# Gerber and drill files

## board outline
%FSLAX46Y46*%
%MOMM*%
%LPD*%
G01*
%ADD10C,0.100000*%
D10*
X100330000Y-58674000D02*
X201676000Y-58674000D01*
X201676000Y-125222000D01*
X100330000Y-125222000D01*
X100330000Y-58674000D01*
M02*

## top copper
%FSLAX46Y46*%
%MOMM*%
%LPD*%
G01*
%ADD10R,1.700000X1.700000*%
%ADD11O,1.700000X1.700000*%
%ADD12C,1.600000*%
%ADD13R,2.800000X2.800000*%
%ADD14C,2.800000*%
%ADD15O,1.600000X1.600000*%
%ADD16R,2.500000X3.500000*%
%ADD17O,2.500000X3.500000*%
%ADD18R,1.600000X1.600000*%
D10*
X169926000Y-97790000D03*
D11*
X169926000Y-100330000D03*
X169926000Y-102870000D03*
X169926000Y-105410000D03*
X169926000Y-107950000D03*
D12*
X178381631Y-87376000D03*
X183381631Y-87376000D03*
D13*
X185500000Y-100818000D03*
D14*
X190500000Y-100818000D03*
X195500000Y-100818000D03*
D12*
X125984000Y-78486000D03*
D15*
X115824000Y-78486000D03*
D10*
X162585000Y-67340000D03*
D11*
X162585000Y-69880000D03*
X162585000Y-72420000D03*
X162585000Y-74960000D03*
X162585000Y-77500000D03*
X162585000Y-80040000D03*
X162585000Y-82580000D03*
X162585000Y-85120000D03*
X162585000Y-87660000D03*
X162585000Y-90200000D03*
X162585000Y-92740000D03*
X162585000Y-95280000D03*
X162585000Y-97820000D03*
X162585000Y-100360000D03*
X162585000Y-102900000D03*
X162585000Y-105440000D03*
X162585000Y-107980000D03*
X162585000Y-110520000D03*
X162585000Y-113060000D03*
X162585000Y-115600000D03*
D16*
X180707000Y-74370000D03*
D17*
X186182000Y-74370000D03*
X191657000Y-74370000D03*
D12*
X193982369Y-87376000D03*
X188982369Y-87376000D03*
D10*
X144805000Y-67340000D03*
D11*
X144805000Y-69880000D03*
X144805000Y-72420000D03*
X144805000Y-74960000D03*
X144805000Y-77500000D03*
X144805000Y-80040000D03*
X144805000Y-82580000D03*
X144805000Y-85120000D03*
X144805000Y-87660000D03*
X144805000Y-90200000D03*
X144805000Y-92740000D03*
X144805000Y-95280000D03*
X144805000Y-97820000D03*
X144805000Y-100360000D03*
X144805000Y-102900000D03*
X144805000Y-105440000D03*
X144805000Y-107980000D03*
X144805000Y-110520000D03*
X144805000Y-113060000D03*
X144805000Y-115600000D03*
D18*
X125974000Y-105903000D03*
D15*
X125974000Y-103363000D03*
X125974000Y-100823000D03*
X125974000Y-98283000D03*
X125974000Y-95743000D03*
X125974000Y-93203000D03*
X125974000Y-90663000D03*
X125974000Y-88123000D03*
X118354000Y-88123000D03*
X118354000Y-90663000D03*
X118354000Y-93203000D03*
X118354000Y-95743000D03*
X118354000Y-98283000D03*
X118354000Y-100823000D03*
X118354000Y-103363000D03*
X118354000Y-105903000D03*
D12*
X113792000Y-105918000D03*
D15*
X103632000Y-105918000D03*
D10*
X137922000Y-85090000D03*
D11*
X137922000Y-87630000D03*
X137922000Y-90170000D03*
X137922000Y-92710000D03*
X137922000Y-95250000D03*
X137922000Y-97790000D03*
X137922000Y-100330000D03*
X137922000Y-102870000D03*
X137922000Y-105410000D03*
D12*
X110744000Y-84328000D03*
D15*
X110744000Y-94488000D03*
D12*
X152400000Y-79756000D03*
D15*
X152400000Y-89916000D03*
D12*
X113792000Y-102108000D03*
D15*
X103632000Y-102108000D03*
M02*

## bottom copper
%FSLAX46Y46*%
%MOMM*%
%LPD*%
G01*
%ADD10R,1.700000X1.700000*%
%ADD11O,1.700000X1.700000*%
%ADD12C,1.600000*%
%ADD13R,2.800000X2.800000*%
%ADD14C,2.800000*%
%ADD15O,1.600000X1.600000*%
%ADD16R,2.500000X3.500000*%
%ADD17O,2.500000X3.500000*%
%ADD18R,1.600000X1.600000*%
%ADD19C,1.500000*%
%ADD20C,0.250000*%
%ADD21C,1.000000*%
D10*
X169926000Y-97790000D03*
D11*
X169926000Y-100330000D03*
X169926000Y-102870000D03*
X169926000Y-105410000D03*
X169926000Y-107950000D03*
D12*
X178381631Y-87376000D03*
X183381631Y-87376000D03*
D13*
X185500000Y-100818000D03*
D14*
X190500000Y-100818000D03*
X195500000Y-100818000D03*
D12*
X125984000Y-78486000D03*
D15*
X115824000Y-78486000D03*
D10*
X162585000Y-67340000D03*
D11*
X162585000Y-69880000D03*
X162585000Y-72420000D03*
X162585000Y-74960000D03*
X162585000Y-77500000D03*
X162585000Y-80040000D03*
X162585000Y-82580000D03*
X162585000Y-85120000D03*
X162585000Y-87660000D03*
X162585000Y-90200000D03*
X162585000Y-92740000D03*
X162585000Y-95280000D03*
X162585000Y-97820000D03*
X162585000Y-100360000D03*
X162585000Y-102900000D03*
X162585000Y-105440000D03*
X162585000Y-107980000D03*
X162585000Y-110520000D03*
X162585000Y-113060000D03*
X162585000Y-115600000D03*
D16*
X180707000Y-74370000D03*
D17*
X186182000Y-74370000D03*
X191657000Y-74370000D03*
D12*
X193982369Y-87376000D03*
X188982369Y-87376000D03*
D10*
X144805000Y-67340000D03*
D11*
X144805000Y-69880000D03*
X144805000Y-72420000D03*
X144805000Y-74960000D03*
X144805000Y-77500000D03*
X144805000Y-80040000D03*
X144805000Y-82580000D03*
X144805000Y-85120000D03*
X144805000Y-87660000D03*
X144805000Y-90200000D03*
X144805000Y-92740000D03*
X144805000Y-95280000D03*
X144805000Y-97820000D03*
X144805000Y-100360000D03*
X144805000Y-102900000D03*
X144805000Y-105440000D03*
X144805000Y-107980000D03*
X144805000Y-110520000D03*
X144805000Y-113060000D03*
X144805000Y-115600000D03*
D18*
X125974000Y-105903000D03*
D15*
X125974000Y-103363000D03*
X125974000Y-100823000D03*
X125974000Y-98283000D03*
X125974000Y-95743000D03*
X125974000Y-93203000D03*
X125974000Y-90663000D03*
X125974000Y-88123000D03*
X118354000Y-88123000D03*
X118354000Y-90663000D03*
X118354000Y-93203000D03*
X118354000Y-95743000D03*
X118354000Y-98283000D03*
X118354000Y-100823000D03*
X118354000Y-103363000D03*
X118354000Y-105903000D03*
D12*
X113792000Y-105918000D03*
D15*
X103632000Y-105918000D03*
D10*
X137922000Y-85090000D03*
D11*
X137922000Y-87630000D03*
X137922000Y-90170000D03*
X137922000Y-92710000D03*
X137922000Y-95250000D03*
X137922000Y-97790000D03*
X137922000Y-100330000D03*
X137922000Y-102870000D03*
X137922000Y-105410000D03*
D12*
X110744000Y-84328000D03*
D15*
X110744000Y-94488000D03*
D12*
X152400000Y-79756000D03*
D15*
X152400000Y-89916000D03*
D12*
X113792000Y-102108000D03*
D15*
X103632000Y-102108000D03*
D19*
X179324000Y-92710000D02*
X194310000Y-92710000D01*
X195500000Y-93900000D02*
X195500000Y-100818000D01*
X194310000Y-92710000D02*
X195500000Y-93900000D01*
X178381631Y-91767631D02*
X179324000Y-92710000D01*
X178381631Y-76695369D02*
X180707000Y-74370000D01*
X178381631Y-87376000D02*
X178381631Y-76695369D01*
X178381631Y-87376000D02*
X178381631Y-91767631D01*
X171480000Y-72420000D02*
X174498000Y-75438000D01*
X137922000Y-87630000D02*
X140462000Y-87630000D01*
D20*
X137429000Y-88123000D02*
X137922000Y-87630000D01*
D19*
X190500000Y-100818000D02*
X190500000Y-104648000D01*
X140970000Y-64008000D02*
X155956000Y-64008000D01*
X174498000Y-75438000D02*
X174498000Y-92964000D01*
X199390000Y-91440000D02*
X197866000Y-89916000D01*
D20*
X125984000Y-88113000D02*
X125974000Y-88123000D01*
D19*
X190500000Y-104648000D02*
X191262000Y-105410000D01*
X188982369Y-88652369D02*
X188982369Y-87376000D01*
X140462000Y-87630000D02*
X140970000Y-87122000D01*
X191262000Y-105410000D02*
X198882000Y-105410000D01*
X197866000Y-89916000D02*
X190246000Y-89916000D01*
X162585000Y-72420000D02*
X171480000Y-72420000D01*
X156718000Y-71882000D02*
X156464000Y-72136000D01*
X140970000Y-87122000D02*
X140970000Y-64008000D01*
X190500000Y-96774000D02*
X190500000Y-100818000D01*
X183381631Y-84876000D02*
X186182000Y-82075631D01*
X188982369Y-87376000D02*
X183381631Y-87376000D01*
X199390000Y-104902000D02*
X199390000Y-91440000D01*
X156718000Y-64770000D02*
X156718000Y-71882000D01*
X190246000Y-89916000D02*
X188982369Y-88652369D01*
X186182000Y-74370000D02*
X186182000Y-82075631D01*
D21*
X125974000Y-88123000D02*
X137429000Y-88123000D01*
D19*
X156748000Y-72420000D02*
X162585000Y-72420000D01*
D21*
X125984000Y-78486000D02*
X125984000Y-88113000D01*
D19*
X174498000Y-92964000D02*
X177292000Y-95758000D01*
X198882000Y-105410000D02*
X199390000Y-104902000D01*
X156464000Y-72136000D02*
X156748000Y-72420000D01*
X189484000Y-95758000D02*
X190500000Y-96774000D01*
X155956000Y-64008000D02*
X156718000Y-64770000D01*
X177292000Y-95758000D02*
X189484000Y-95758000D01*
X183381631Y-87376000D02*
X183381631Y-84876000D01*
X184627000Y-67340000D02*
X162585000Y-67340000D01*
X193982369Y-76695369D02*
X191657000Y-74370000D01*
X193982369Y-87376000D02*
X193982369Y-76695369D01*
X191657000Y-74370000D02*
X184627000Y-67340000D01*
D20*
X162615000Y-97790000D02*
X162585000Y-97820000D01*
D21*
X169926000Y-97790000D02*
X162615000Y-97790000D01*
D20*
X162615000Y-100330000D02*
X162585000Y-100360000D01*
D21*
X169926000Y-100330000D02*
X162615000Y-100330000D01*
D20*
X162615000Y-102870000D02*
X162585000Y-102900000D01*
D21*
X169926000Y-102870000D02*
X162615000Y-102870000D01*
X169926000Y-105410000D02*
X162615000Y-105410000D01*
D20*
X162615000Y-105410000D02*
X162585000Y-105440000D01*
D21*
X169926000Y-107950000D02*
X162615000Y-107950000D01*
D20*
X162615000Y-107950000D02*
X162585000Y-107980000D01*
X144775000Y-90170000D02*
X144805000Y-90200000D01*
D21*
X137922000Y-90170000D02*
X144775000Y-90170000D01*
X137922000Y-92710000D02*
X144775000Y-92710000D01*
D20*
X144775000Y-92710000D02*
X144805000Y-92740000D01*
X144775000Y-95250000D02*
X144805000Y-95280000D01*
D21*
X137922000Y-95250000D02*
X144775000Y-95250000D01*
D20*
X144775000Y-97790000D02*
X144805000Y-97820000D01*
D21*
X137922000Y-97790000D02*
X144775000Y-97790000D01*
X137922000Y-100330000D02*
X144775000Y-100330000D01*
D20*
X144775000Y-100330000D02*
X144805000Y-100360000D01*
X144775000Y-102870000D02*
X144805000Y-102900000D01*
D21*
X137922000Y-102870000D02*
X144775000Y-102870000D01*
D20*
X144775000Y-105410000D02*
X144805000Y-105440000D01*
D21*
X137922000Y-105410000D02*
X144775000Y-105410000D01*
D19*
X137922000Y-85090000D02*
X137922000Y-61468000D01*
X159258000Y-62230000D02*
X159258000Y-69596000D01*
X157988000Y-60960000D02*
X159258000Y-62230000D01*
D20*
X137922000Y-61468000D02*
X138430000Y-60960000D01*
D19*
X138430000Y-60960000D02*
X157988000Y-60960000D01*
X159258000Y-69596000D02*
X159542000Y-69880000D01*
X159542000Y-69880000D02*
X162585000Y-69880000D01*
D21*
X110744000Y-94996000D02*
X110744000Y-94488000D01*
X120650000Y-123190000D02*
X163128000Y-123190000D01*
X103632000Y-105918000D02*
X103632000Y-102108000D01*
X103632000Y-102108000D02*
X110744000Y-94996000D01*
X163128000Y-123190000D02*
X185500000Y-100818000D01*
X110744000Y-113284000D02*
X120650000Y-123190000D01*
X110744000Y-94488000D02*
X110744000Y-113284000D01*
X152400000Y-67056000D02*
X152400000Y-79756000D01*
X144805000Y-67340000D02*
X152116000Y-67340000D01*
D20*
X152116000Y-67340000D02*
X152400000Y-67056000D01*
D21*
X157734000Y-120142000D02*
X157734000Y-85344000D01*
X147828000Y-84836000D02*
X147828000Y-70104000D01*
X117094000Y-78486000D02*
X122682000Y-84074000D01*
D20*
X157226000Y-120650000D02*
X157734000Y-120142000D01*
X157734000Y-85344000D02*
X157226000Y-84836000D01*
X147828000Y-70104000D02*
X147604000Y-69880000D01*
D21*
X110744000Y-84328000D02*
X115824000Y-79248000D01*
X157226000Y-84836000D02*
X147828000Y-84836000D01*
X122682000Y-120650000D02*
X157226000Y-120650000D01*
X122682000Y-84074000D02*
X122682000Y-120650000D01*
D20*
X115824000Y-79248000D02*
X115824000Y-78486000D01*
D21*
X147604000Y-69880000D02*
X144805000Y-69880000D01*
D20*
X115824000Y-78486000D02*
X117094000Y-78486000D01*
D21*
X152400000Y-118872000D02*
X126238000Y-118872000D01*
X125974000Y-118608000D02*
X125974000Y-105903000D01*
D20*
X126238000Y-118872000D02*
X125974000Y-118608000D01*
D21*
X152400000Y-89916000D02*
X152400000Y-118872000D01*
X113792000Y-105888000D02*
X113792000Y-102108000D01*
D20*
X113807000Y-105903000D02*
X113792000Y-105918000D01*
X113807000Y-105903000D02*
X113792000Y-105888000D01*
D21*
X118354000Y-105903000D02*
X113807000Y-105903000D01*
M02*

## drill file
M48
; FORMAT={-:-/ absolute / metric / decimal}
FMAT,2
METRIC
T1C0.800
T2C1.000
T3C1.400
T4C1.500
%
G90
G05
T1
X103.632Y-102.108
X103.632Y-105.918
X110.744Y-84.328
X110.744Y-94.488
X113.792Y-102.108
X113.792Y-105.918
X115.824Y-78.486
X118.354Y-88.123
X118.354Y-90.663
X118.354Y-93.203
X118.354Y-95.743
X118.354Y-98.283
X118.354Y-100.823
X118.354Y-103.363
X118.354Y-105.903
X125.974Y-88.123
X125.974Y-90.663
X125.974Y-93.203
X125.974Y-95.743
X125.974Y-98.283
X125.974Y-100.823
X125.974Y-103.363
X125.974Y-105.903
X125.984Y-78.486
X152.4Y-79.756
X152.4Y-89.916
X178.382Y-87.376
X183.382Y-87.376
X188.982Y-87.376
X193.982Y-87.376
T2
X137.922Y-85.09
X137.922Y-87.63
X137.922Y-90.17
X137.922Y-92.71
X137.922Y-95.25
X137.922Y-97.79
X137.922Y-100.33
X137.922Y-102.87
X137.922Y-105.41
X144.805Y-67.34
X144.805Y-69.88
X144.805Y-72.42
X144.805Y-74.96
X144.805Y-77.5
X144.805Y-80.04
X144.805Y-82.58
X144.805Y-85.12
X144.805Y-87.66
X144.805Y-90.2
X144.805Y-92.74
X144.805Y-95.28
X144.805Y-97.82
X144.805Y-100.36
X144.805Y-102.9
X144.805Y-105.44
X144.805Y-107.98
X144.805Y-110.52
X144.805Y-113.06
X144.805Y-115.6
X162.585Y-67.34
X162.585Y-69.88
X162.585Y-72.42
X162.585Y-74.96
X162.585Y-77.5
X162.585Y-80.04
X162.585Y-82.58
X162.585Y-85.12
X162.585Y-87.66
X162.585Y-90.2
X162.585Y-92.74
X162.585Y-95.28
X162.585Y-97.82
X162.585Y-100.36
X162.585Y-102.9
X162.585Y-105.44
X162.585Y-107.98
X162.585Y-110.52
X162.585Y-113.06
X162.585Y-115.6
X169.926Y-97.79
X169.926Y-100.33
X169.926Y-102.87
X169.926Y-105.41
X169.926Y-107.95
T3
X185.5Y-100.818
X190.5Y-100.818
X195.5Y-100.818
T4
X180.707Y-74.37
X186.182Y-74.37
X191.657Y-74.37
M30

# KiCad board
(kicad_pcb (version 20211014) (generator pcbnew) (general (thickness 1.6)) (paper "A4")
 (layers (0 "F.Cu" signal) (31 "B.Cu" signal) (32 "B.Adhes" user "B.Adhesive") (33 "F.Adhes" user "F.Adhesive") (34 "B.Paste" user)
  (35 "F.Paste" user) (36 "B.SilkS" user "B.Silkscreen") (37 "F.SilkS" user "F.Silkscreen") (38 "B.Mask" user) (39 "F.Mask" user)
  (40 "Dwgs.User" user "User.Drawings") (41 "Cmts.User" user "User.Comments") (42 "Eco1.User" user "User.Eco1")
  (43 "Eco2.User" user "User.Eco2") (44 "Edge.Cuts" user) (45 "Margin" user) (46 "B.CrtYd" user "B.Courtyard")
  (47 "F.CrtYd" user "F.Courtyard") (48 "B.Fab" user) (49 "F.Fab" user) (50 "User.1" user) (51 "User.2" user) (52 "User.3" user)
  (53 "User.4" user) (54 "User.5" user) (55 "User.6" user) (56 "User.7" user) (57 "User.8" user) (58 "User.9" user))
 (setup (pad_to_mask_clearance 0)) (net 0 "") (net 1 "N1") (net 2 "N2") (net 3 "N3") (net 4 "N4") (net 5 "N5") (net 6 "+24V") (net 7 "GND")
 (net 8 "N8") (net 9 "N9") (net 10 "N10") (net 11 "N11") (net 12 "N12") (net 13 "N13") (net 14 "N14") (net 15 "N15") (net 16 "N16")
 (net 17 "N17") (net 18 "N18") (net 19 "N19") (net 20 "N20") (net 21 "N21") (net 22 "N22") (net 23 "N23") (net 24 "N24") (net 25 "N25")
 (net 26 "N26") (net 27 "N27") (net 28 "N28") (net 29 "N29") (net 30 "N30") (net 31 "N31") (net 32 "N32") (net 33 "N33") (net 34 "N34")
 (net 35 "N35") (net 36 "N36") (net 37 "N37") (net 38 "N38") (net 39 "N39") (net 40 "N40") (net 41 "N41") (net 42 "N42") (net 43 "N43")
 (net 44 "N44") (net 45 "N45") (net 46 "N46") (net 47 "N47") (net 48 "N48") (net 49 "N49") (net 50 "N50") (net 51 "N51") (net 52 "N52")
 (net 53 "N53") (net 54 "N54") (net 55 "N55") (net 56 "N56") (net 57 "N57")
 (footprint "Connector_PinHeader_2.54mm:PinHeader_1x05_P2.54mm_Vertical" (layer "F.Cu") (at 169.926 97.79)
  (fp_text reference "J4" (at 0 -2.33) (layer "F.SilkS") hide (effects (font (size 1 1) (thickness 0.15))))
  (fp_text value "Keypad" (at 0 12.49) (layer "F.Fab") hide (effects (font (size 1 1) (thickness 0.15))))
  (pad "1" thru_hole rect (at 0 0) (size 1.7 1.7) (drill 1) (layers *.Cu *.Mask) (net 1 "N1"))
  (pad "2" thru_hole oval (at 0 2.54) (size 1.7 1.7) (drill 1) (layers *.Cu *.Mask) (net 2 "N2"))
  (pad "3" thru_hole oval (at 0 5.08) (size 1.7 1.7) (drill 1) (layers *.Cu *.Mask) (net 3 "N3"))
  (pad "4" thru_hole oval (at 0 7.62) (size 1.7 1.7) (drill 1) (layers *.Cu *.Mask) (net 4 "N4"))
  (pad "5" thru_hole oval (at 0 10.16) (size 1.7 1.7) (drill 1) (layers *.Cu *.Mask) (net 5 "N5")))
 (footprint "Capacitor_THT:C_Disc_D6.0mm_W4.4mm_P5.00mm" (layer "F.Cu") (at 178.381631 87.376)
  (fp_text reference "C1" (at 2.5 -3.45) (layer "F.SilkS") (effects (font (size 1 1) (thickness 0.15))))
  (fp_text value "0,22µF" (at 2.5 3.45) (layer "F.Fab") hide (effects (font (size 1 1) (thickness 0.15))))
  (pad "1" thru_hole circle (at 0 0) (size 1.6 1.6) (drill 0.8) (layers *.Cu *.Mask) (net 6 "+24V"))
  (pad "2" thru_hole circle (at 5 0) (size 1.6 1.6) (drill 0.8) (layers *.Cu *.Mask) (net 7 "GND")))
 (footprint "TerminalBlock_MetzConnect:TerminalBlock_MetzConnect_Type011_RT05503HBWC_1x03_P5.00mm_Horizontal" (layer "F.Cu")
  (at 185.5 100.818)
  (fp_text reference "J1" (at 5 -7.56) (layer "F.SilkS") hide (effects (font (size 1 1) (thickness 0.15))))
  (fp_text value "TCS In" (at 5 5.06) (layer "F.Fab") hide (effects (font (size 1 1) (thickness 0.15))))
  (pad "1" thru_hole rect (at 0 0) (size 2.8 2.8) (drill 1.4) (layers *.Cu *.Mask) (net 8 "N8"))
  (pad "2" thru_hole circle (at 5 0) (size 2.8 2.8) (drill 1.4) (layers *.Cu *.Mask) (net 7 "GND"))
  (pad "3" thru_hole circle (at 10 0) (size 2.8 2.8) (drill 1.4) (layers *.Cu *.Mask) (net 6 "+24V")))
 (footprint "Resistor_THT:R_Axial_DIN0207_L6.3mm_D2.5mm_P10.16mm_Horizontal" (layer "F.Cu") (at 125.984 78.486 180)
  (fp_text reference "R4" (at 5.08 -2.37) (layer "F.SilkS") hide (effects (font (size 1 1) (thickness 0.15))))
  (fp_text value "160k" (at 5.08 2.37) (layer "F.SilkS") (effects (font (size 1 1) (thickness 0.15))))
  (pad "1" thru_hole circle (at 0 0 180) (size 1.6 1.6) (drill 0.8) (layers *.Cu *.Mask) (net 7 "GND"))
  (pad "2" thru_hole oval (at 10.16 0 180) (size 1.6 1.6) (drill 0.8) (layers *.Cu *.Mask) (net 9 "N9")))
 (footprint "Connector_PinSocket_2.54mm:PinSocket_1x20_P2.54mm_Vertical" (layer "F.Cu") (at 162.585 67.34)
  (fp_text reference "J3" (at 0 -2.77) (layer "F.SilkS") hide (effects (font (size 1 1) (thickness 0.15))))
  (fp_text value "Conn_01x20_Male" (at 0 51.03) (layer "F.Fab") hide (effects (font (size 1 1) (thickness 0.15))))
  (pad "1" thru_hole rect (at 0 0) (size 1.7 1.7) (drill 1) (layers *.Cu *.Mask) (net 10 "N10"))
  (pad "2" thru_hole oval (at 0 2.54) (size 1.7 1.7) (drill 1) (layers *.Cu *.Mask) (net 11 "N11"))
  (pad "3" thru_hole oval (at 0 5.08) (size 1.7 1.7) (drill 1) (layers *.Cu *.Mask) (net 7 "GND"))
  (pad "4" thru_hole oval (at 0 7.62) (size 1.7 1.7) (drill 1) (layers *.Cu *.Mask) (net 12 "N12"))
  (pad "5" thru_hole oval (at 0 10.16) (size 1.7 1.7) (drill 1) (layers *.Cu *.Mask) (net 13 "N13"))
  (pad "6" thru_hole oval (at 0 12.7) (size 1.7 1.7) (drill 1) (layers *.Cu *.Mask) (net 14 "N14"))
  (pad "7" thru_hole oval (at 0 15.24) (size 1.7 1.7) (drill 1) (layers *.Cu *.Mask) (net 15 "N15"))
  (pad "8" thru_hole oval (at 0 17.78) (size 1.7 1.7) (drill 1) (layers *.Cu *.Mask) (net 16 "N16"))
  (pad "9" thru_hole oval (at 0 20.32) (size 1.7 1.7) (drill 1) (layers *.Cu *.Mask) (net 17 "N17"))
  (pad "10" thru_hole oval (at 0 22.86) (size 1.7 1.7) (drill 1) (layers *.Cu *.Mask) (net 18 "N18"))
  (pad "11" thru_hole oval (at 0 25.4) (size 1.7 1.7) (drill 1) (layers *.Cu *.Mask) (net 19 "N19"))
  (pad "12" thru_hole oval (at 0 27.94) (size 1.7 1.7) (drill 1) (layers *.Cu *.Mask) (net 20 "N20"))
  (pad "13" thru_hole oval (at 0 30.48) (size 1.7 1.7) (drill 1) (layers *.Cu *.Mask) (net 1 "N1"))
  (pad "14" thru_hole oval (at 0 33.02) (size 1.7 1.7) (drill 1) (layers *.Cu *.Mask) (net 2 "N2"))
  (pad "15" thru_hole oval (at 0 35.56) (size 1.7 1.7) (drill 1) (layers *.Cu *.Mask) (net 3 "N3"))
  (pad "16" thru_hole oval (at 0 38.1) (size 1.7 1.7) (drill 1) (layers *.Cu *.Mask) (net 4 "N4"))
  (pad "17" thru_hole oval (at 0 40.64) (size 1.7 1.7) (drill 1) (layers *.Cu *.Mask) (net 5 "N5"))
  (pad "18" thru_hole oval (at 0 43.18) (size 1.7 1.7) (drill 1) (layers *.Cu *.Mask) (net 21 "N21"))
  (pad "19" thru_hole oval (at 0 45.72) (size 1.7 1.7) (drill 1) (layers *.Cu *.Mask) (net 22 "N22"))
  (pad "20" thru_hole oval (at 0 48.26) (size 1.7 1.7) (drill 1) (layers *.Cu *.Mask) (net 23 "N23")))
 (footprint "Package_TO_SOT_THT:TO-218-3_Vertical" (layer "F.Cu") (at 180.707 74.37)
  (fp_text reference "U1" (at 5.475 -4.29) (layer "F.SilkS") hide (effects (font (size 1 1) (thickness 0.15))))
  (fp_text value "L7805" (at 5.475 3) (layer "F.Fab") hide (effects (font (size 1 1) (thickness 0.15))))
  (pad "1" thru_hole rect (at 0 0) (size 2.5 3.5) (drill 1.5) (layers *.Cu *.Mask) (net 6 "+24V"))
  (pad "2" thru_hole oval (at 5.475 0) (size 2.5 3.5) (drill 1.5) (layers *.Cu *.Mask) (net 7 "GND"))
  (pad "3" thru_hole oval (at 10.95 0) (size 2.5 3.5) (drill 1.5) (layers *.Cu *.Mask) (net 10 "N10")))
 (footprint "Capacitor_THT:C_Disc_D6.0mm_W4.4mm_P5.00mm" (layer "F.Cu") (at 193.982369 87.376 180)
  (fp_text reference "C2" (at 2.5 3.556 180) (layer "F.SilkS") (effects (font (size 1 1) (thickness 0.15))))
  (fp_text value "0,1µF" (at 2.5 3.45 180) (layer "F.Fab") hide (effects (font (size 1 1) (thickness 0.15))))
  (pad "1" thru_hole circle (at 0 0 180) (size 1.6 1.6) (drill 0.8) (layers *.Cu *.Mask) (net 10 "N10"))
  (pad "2" thru_hole circle (at 5 0 180) (size 1.6 1.6) (drill 0.8) (layers *.Cu *.Mask) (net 7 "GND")))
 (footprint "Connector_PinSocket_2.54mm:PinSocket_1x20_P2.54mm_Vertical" (layer "F.Cu") (at 144.805 67.34)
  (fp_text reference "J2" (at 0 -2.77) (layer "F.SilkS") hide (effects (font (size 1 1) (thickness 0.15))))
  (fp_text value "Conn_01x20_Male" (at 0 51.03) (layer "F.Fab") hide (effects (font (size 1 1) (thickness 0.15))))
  (pad "1" thru_hole rect (at 0 0) (size 1.7 1.7) (drill 1) (layers *.Cu *.Mask) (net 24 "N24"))
  (pad "2" thru_hole oval (at 0 2.54) (size 1.7 1.7) (drill 1) (layers *.Cu *.Mask) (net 9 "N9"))
  (pad "3" thru_hole oval (at 0 5.08) (size 1.7 1.7) (drill 1) (layers *.Cu *.Mask) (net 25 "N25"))
  (pad "4" thru_hole oval (at 0 7.62) (size 1.7 1.7) (drill 1) (layers *.Cu *.Mask) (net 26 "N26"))
  (pad "5" thru_hole oval (at 0 10.16) (size 1.7 1.7) (drill 1) (layers *.Cu *.Mask) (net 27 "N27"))
  (pad "6" thru_hole oval (at 0 12.7) (size 1.7 1.7) (drill 1) (layers *.Cu *.Mask) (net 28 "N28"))
  (pad "7" thru_hole oval (at 0 15.24) (size 1.7 1.7) (drill 1) (layers *.Cu *.Mask) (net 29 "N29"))
  (pad "8" thru_hole oval (at 0 17.78) (size 1.7 1.7) (drill 1) (layers *.Cu *.Mask) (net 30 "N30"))
  (pad "9" thru_hole oval (at 0 20.32) (size 1.7 1.7) (drill 1) (layers *.Cu *.Mask) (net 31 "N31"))
  (pad "10" thru_hole oval (at 0 22.86) (size 1.7 1.7) (drill 1) (layers *.Cu *.Mask) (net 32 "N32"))
  (pad "11" thru_hole oval (at 0 25.4) (size 1.7 1.7) (drill 1) (layers *.Cu *.Mask) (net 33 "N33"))
  (pad "12" thru_hole oval (at 0 27.94) (size 1.7 1.7) (drill 1) (layers *.Cu *.Mask) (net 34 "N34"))
  (pad "13" thru_hole oval (at 0 30.48) (size 1.7 1.7) (drill 1) (layers *.Cu *.Mask) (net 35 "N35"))
  (pad "14" thru_hole oval (at 0 33.02) (size 1.7 1.7) (drill 1) (layers *.Cu *.Mask) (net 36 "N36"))
  (pad "15" thru_hole oval (at 0 35.56) (size 1.7 1.7) (drill 1) (layers *.Cu *.Mask) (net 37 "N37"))
  (pad "16" thru_hole oval (at 0 38.1) (size 1.7 1.7) (drill 1) (layers *.Cu *.Mask) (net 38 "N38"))
  (pad "17" thru_hole oval (at 0 40.64) (size 1.7 1.7) (drill 1) (layers *.Cu *.Mask) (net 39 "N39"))
  (pad "18" thru_hole oval (at 0 43.18) (size 1.7 1.7) (drill 1) (layers *.Cu *.Mask) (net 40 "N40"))
  (pad "19" thru_hole oval (at 0 45.72) (size 1.7 1.7) (drill 1) (layers *.Cu *.Mask) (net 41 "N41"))
  (pad "20" thru_hole oval (at 0 48.26) (size 1.7 1.7) (drill 1) (layers *.Cu *.Mask) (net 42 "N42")))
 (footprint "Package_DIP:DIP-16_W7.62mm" (layer "F.Cu") (at 125.974 105.903 180)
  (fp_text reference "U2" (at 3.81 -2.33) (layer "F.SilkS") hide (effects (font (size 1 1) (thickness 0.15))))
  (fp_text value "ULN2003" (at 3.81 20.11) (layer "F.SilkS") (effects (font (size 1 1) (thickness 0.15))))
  (pad "1" thru_hole rect (at 0 0 180) (size 1.6 1.6) (drill 0.8) (layers *.Cu *.Mask) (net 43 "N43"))
  (pad "2" thru_hole oval (at 0 2.54 180) (size 1.6 1.6) (drill 0.8) (layers *.Cu *.Mask) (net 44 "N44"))
  (pad "3" thru_hole oval (at 0 5.08 180) (size 1.6 1.6) (drill 0.8) (layers *.Cu *.Mask) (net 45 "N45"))
  (pad "4" thru_hole oval (at 0 7.62 180) (size 1.6 1.6) (drill 0.8) (layers *.Cu *.Mask) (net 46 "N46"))
  (pad "5" thru_hole oval (at 0 10.16 180) (size 1.6 1.6) (drill 0.8) (layers *.Cu *.Mask) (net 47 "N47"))
  (pad "6" thru_hole oval (at 0 12.7 180) (size 1.6 1.6) (drill 0.8) (layers *.Cu *.Mask) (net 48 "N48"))
  (pad "7" thru_hole oval (at 0 15.24 180) (size 1.6 1.6) (drill 0.8) (layers *.Cu *.Mask) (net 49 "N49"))
  (pad "8" thru_hole oval (at 0 17.78 180) (size 1.6 1.6) (drill 0.8) (layers *.Cu *.Mask) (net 7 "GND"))
  (pad "9" thru_hole oval (at 7.62 17.78 180) (size 1.6 1.6) (drill 0.8) (layers *.Cu *.Mask) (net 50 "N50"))
  (pad "10" thru_hole oval (at 7.62 15.24 180) (size 1.6 1.6) (drill 0.8) (layers *.Cu *.Mask) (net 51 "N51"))
  (pad "11" thru_hole oval (at 7.62 12.7 180) (size 1.6 1.6) (drill 0.8) (layers *.Cu *.Mask) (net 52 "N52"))
  (pad "12" thru_hole oval (at 7.62 10.16 180) (size 1.6 1.6) (drill 0.8) (layers *.Cu *.Mask) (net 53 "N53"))
  (pad "13" thru_hole oval (at 7.62 7.62 180) (size 1.6 1.6) (drill 0.8) (layers *.Cu *.Mask) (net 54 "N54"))
  (pad "14" thru_hole oval (at 7.62 5.08 180) (size 1.6 1.6) (drill 0.8) (layers *.Cu *.Mask) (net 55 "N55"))
  (pad "15" thru_hole oval (at 7.62 2.54 180) (size 1.6 1.6) (drill 0.8) (layers *.Cu *.Mask) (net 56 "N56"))
  (pad "16" thru_hole oval (at 7.62 0 180) (size 1.6 1.6) (drill 0.8) (layers *.Cu *.Mask) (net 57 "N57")))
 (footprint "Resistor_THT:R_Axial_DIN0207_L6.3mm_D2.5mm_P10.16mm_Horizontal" (layer "F.Cu") (at 113.792 105.918 180)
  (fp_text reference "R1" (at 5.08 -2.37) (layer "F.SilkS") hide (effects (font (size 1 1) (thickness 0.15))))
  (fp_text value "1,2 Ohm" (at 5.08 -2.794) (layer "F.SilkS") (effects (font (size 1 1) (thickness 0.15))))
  (pad "1" thru_hole circle (at 0 0 180) (size 1.6 1.6) (drill 0.8) (layers *.Cu *.Mask) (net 57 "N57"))
  (pad "2" thru_hole oval (at 10.16 0 180) (size 1.6 1.6) (drill 0.8) (layers *.Cu *.Mask) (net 8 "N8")))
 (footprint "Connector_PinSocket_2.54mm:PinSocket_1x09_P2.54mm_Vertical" (layer "F.Cu") (at 137.922 85.09)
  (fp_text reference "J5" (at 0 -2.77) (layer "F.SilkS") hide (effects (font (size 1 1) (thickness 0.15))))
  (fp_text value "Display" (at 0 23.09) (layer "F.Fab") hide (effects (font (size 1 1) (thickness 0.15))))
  (pad "1" thru_hole rect (at 0 0) (size 1.7 1.7) (drill 1) (layers *.Cu *.Mask) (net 11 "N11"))
  (pad "2" thru_hole oval (at 0 2.54) (size 1.7 1.7) (drill 1) (layers *.Cu *.Mask) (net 7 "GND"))
  (pad "3" thru_hole oval (at 0 5.08) (size 1.7 1.7) (drill 1) (layers *.Cu *.Mask) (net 32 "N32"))
  (pad "4" thru_hole oval (at 0 7.62) (size 1.7 1.7) (drill 1) (layers *.Cu *.Mask) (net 33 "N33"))
  (pad "5" thru_hole oval (at 0 10.16) (size 1.7 1.7) (drill 1) (layers *.Cu *.Mask) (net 34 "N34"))
  (pad "6" thru_hole oval (at 0 12.7) (size 1.7 1.7) (drill 1) (layers *.Cu *.Mask) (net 35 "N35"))
  (pad "7" thru_hole oval (at 0 15.24) (size 1.7 1.7) (drill 1) (layers *.Cu *.Mask) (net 36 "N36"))
  (pad "8" thru_hole oval (at 0 17.78) (size 1.7 1.7) (drill 1) (layers *.Cu *.Mask) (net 37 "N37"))
  (pad "9" thru_hole oval (at 0 20.32) (size 1.7 1.7) (drill 1) (layers *.Cu *.Mask) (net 38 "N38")))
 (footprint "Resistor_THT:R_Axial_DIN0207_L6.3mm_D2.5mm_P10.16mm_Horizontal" (layer "F.Cu") (at 110.744 84.328 -90)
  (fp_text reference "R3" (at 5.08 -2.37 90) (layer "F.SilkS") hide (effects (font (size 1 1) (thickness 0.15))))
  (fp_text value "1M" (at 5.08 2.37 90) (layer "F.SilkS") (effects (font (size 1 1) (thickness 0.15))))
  (pad "1" thru_hole circle (at 0 0 270) (size 1.6 1.6) (drill 0.8) (layers *.Cu *.Mask) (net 9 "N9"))
  (pad "2" thru_hole oval (at 10.16 0 270) (size 1.6 1.6) (drill 0.8) (layers *.Cu *.Mask) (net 8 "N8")))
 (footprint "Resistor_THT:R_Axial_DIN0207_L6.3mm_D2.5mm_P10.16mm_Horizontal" (layer "F.Cu") (at 152.4 79.756 -90)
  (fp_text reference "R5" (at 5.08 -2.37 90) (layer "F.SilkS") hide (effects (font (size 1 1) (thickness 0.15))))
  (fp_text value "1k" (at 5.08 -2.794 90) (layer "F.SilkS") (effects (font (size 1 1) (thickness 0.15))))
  (pad "1" thru_hole circle (at 0 0 270) (size 1.6 1.6) (drill 0.8) (layers *.Cu *.Mask) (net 24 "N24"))
  (pad "2" thru_hole oval (at 10.16 0 270) (size 1.6 1.6) (drill 0.8) (layers *.Cu *.Mask) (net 43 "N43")))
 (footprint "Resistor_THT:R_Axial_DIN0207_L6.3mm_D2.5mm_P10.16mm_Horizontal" (layer "F.Cu") (at 113.792 102.108 180)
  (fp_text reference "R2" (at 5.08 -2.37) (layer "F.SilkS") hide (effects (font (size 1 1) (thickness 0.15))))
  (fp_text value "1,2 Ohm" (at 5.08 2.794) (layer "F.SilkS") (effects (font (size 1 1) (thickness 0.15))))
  (pad "1" thru_hole circle (at 0 0 180) (size 1.6 1.6) (drill 0.8) (layers *.Cu *.Mask) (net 57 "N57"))
  (pad "2" thru_hole oval (at 10.16 0 180) (size 1.6 1.6) (drill 0.8) (layers *.Cu *.Mask) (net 8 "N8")))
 (gr_rect (start 100.33 58.674) (end 201.676 125.222) (layer "Edge.Cuts") (width 0.1) (fill none))
 (segment (start 179.324 92.71) (end 194.31 92.71) (width 1.5) (layer "B.Cu") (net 6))
 (segment (start 195.5 93.9) (end 195.5 100.818) (width 1.5) (layer "B.Cu") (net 6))
 (segment (start 194.31 92.71) (end 195.5 93.9) (width 1.5) (layer "B.Cu") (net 6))
 (segment (start 178.381631 91.767631) (end 179.324 92.71) (width 1.5) (layer "B.Cu") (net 6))
 (segment (start 178.381631 76.695369) (end 180.707 74.37) (width 1.5) (layer "B.Cu") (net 6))
 (segment (start 178.381631 87.376) (end 178.381631 76.695369) (width 1.5) (layer "B.Cu") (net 6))
 (segment (start 178.381631 87.376) (end 178.381631 91.767631) (width 1.5) (layer "B.Cu") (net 6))
 (segment (start 171.48 72.42) (end 174.498 75.438) (width 1.5) (layer "B.Cu") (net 7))
 (segment (start 137.922 87.63) (end 140.462 87.63) (width 1.5) (layer "B.Cu") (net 7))
 (segment (start 137.429 88.123) (end 137.922 87.63) (width 0.25) (layer "B.Cu") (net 7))
 (segment (start 190.5 100.818) (end 190.5 104.648) (width 1.5) (layer "B.Cu") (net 7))
 (segment (start 140.97 64.008) (end 155.956 64.008) (width 1.5) (layer "B.Cu") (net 7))
 (segment (start 174.498 75.438) (end 174.498 92.964) (width 1.5) (layer "B.Cu") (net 7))
 (segment (start 199.39 91.44) (end 197.866 89.916) (width 1.5) (layer "B.Cu") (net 7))
 (segment (start 125.984 88.113) (end 125.974 88.123) (width 0.25) (layer "B.Cu") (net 7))
 (segment (start 190.5 104.648) (end 191.262 105.41) (width 1.5) (layer "B.Cu") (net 7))
 (segment (start 188.982369 88.652369) (end 188.982369 87.376) (width 1.5) (layer "B.Cu") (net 7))
 (segment (start 140.462 87.63) (end 140.97 87.122) (width 1.5) (layer "B.Cu") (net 7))
 (segment (start 191.262 105.41) (end 198.882 105.41) (width 1.5) (layer "B.Cu") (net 7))
 (segment (start 197.866 89.916) (end 190.246 89.916) (width 1.5) (layer "B.Cu") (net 7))
 (segment (start 162.585 72.42) (end 171.48 72.42) (width 1.5) (layer "B.Cu") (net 7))
 (segment (start 156.718 71.882) (end 156.464 72.136) (width 1.5) (layer "B.Cu") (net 7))
 (segment (start 140.97 87.122) (end 140.97 64.008) (width 1.5) (layer "B.Cu") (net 7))
 (segment (start 190.5 96.774) (end 190.5 100.818) (width 1.5) (layer "B.Cu") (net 7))
 (segment (start 183.381631 84.876) (end 186.182 82.075631) (width 1.5) (layer "B.Cu") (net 7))
 (segment (start 188.982369 87.376) (end 183.381631 87.376) (width 1.5) (layer "B.Cu") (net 7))
 (segment (start 199.39 104.902) (end 199.39 91.44) (width 1.5) (layer "B.Cu") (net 7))
 (segment (start 156.718 64.77) (end 156.718 71.882) (width 1.5) (layer "B.Cu") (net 7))
 (segment (start 190.246 89.916) (end 188.982369 88.652369) (width 1.5) (layer "B.Cu") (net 7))
 (segment (start 186.182 74.37) (end 186.182 82.075631) (width 1.5) (layer "B.Cu") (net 7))
 (segment (start 125.974 88.123) (end 137.429 88.123) (width 1) (layer "B.Cu") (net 7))
 (segment (start 156.748 72.42) (end 162.585 72.42) (width 1.5) (layer "B.Cu") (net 7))
 (segment (start 125.984 78.486) (end 125.984 88.113) (width 1) (layer "B.Cu") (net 7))
 (segment (start 174.498 92.964) (end 177.292 95.758) (width 1.5) (layer "B.Cu") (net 7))
 (segment (start 198.882 105.41) (end 199.39 104.902) (width 1.5) (layer "B.Cu") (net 7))
 (segment (start 156.464 72.136) (end 156.748 72.42) (width 1.5) (layer "B.Cu") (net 7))
 (segment (start 189.484 95.758) (end 190.5 96.774) (width 1.5) (layer "B.Cu") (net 7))
 (segment (start 155.956 64.008) (end 156.718 64.77) (width 1.5) (layer "B.Cu") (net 7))
 (segment (start 177.292 95.758) (end 189.484 95.758) (width 1.5) (layer "B.Cu") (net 7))
 (segment (start 183.381631 87.376) (end 183.381631 84.876) (width 1.5) (layer "B.Cu") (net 7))
 (segment (start 184.627 67.34) (end 162.585 67.34) (width 1.5) (layer "B.Cu") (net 10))
 (segment (start 193.982369 76.695369) (end 191.657 74.37) (width 1.5) (layer "B.Cu") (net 10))
 (segment (start 193.982369 87.376) (end 193.982369 76.695369) (width 1.5) (layer "B.Cu") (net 10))
 (segment (start 191.657 74.37) (end 184.627 67.34) (width 1.5) (layer "B.Cu") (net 10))
 (segment (start 162.615 97.79) (end 162.585 97.82) (width 0.25) (layer "B.Cu") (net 1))
 (segment (start 169.926 97.79) (end 162.615 97.79) (width 1) (layer "B.Cu") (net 1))
 (segment (start 162.615 100.33) (end 162.585 100.36) (width 0.25) (layer "B.Cu") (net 2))
 (segment (start 169.926 100.33) (end 162.615 100.33) (width 1) (layer "B.Cu") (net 2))
 (segment (start 162.615 102.87) (end 162.585 102.9) (width 0.25) (layer "B.Cu") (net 3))
 (segment (start 169.926 102.87) (end 162.615 102.87) (width 1) (layer "B.Cu") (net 3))
 (segment (start 169.926 105.41) (end 162.615 105.41) (width 1) (layer "B.Cu") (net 4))
 (segment (start 162.615 105.41) (end 162.585 105.44) (width 0.25) (layer "B.Cu") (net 4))
 (segment (start 169.926 107.95) (end 162.615 107.95) (width 1) (layer "B.Cu") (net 5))
 (segment (start 162.615 107.95) (end 162.585 107.98) (width 0.25) (layer "B.Cu") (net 5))
 (segment (start 144.775 90.17) (end 144.805 90.2) (width 0.25) (layer "B.Cu") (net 32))
 (segment (start 137.922 90.17) (end 144.775 90.17) (width 1) (layer "B.Cu") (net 32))
 (segment (start 137.922 92.71) (end 144.775 92.71) (width 1) (layer "B.Cu") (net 33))
 (segment (start 144.775 92.71) (end 144.805 92.74) (width 0.25) (layer "B.Cu") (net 33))
 (segment (start 144.775 95.25) (end 144.805 95.28) (width 0.25) (layer "B.Cu") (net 34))
 (segment (start 137.922 95.25) (end 144.775 95.25) (width 1) (layer "B.Cu") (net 34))
 (segment (start 144.775 97.79) (end 144.805 97.82) (width 0.25) (layer "B.Cu") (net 35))
 (segment (start 137.922 97.79) (end 144.775 97.79) (width 1) (layer "B.Cu") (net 35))
 (segment (start 137.922 100.33) (end 144.775 100.33) (width 1) (layer "B.Cu") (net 36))
 (segment (start 144.775 100.33) (end 144.805 100.36) (width 0.25) (layer "B.Cu") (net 36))
 (segment (start 144.775 102.87) (end 144.805 102.9) (width 0.25) (layer "B.Cu") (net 37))
 (segment (start 137.922 102.87) (end 144.775 102.87) (width 1) (layer "B.Cu") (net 37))
 (segment (start 144.775 105.41) (end 144.805 105.44) (width 0.25) (layer "B.Cu") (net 38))
 (segment (start 137.922 105.41) (end 144.775 105.41) (width 1) (layer "B.Cu") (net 38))
 (segment (start 137.922 85.09) (end 137.922 61.468) (width 1.5) (layer "B.Cu") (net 11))
 (segment (start 159.258 62.23) (end 159.258 69.596) (width 1.5) (layer "B.Cu") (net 11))
 (segment (start 157.988 60.96) (end 159.258 62.23) (width 1.5) (layer "B.Cu") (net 11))
 (segment (start 137.922 61.468) (end 138.43 60.96) (width 0.25) (layer "B.Cu") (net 11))
 (segment (start 138.43 60.96) (end 157.988 60.96) (width 1.5) (layer "B.Cu") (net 11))
 (segment (start 159.258 69.596) (end 159.542 69.88) (width 1.5) (layer "B.Cu") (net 11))
 (segment (start 159.542 69.88) (end 162.585 69.88) (width 1.5) (layer "B.Cu") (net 11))
 (segment (start 110.744 94.996) (end 110.744 94.488) (width 1) (layer "B.Cu") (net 8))
 (segment (start 120.65 123.19) (end 163.128 123.19) (width 1) (layer "B.Cu") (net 8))
 (segment (start 103.632 105.918) (end 103.632 102.108) (width 1) (layer "B.Cu") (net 8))
 (segment (start 103.632 102.108) (end 110.744 94.996) (width 1) (layer "B.Cu") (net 8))
 (segment (start 163.128 123.19) (end 185.5 100.818) (width 1) (layer "B.Cu") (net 8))
 (segment (start 110.744 113.284) (end 120.65 123.19) (width 1) (layer "B.Cu") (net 8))
 (segment (start 110.744 94.488) (end 110.744 113.284) (width 1) (layer "B.Cu") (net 8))
 (segment (start 152.4 67.056) (end 152.4 79.756) (width 1) (layer "B.Cu") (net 24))
 (segment (start 144.805 67.34) (end 152.116 67.34) (width 1) (layer "B.Cu") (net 24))
 (segment (start 152.116 67.34) (end 152.4 67.056) (width 0.25) (layer "B.Cu") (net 24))
 (segment (start 157.734 120.142) (end 157.734 85.344) (width 1) (layer "B.Cu") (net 9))
 (segment (start 147.828 84.836) (end 147.828 70.104) (width 1) (layer "B.Cu") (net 9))
 (segment (start 117.094 78.486) (end 122.682 84.074) (width 1) (layer "B.Cu") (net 9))
 (segment (start 157.226 120.65) (end 157.734 120.142) (width 0.25) (layer "B.Cu") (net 9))
 (segment (start 157.734 85.344) (end 157.226 84.836) (width 0.25) (layer "B.Cu") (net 9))
 (segment (start 147.828 70.104) (end 147.604 69.88) (width 0.25) (layer "B.Cu") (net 9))
 (segment (start 110.744 84.328) (end 115.824 79.248) (width 1) (layer "B.Cu") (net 9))
 (segment (start 157.226 84.836) (end 147.828 84.836) (width 1) (layer "B.Cu") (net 9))
 (segment (start 122.682 120.65) (end 157.226 120.65) (width 1) (layer "B.Cu") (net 9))
 (segment (start 122.682 84.074) (end 122.682 120.65) (width 1) (layer "B.Cu") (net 9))
 (segment (start 115.824 79.248) (end 115.824 78.486) (width 0.25) (layer "B.Cu") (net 9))
 (segment (start 147.604 69.88) (end 144.805 69.88) (width 1) (layer "B.Cu") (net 9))
 (segment (start 115.824 78.486) (end 117.094 78.486) (width 0.25) (layer "B.Cu") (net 9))
 (segment (start 152.4 118.872) (end 126.238 118.872) (width 1) (layer "B.Cu") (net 43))
 (segment (start 125.974 118.608) (end 125.974 105.903) (width 1) (layer "B.Cu") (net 43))
 (segment (start 126.238 118.872) (end 125.974 118.608) (width 0.25) (layer "B.Cu") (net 43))
 (segment (start 152.4 89.916) (end 152.4 118.872) (width 1) (layer "B.Cu") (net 43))
 (segment (start 113.792 105.888) (end 113.792 102.108) (width 1) (layer "B.Cu") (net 57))
 (segment (start 113.807 105.903) (end 113.792 105.918) (width 0.25) (layer "B.Cu") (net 57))
 (segment (start 113.807 105.903) (end 113.792 105.888) (width 0.25) (layer "B.Cu") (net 57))
 (segment (start 118.354 105.903) (end 113.807 105.903) (width 1) (layer "B.Cu") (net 57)))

